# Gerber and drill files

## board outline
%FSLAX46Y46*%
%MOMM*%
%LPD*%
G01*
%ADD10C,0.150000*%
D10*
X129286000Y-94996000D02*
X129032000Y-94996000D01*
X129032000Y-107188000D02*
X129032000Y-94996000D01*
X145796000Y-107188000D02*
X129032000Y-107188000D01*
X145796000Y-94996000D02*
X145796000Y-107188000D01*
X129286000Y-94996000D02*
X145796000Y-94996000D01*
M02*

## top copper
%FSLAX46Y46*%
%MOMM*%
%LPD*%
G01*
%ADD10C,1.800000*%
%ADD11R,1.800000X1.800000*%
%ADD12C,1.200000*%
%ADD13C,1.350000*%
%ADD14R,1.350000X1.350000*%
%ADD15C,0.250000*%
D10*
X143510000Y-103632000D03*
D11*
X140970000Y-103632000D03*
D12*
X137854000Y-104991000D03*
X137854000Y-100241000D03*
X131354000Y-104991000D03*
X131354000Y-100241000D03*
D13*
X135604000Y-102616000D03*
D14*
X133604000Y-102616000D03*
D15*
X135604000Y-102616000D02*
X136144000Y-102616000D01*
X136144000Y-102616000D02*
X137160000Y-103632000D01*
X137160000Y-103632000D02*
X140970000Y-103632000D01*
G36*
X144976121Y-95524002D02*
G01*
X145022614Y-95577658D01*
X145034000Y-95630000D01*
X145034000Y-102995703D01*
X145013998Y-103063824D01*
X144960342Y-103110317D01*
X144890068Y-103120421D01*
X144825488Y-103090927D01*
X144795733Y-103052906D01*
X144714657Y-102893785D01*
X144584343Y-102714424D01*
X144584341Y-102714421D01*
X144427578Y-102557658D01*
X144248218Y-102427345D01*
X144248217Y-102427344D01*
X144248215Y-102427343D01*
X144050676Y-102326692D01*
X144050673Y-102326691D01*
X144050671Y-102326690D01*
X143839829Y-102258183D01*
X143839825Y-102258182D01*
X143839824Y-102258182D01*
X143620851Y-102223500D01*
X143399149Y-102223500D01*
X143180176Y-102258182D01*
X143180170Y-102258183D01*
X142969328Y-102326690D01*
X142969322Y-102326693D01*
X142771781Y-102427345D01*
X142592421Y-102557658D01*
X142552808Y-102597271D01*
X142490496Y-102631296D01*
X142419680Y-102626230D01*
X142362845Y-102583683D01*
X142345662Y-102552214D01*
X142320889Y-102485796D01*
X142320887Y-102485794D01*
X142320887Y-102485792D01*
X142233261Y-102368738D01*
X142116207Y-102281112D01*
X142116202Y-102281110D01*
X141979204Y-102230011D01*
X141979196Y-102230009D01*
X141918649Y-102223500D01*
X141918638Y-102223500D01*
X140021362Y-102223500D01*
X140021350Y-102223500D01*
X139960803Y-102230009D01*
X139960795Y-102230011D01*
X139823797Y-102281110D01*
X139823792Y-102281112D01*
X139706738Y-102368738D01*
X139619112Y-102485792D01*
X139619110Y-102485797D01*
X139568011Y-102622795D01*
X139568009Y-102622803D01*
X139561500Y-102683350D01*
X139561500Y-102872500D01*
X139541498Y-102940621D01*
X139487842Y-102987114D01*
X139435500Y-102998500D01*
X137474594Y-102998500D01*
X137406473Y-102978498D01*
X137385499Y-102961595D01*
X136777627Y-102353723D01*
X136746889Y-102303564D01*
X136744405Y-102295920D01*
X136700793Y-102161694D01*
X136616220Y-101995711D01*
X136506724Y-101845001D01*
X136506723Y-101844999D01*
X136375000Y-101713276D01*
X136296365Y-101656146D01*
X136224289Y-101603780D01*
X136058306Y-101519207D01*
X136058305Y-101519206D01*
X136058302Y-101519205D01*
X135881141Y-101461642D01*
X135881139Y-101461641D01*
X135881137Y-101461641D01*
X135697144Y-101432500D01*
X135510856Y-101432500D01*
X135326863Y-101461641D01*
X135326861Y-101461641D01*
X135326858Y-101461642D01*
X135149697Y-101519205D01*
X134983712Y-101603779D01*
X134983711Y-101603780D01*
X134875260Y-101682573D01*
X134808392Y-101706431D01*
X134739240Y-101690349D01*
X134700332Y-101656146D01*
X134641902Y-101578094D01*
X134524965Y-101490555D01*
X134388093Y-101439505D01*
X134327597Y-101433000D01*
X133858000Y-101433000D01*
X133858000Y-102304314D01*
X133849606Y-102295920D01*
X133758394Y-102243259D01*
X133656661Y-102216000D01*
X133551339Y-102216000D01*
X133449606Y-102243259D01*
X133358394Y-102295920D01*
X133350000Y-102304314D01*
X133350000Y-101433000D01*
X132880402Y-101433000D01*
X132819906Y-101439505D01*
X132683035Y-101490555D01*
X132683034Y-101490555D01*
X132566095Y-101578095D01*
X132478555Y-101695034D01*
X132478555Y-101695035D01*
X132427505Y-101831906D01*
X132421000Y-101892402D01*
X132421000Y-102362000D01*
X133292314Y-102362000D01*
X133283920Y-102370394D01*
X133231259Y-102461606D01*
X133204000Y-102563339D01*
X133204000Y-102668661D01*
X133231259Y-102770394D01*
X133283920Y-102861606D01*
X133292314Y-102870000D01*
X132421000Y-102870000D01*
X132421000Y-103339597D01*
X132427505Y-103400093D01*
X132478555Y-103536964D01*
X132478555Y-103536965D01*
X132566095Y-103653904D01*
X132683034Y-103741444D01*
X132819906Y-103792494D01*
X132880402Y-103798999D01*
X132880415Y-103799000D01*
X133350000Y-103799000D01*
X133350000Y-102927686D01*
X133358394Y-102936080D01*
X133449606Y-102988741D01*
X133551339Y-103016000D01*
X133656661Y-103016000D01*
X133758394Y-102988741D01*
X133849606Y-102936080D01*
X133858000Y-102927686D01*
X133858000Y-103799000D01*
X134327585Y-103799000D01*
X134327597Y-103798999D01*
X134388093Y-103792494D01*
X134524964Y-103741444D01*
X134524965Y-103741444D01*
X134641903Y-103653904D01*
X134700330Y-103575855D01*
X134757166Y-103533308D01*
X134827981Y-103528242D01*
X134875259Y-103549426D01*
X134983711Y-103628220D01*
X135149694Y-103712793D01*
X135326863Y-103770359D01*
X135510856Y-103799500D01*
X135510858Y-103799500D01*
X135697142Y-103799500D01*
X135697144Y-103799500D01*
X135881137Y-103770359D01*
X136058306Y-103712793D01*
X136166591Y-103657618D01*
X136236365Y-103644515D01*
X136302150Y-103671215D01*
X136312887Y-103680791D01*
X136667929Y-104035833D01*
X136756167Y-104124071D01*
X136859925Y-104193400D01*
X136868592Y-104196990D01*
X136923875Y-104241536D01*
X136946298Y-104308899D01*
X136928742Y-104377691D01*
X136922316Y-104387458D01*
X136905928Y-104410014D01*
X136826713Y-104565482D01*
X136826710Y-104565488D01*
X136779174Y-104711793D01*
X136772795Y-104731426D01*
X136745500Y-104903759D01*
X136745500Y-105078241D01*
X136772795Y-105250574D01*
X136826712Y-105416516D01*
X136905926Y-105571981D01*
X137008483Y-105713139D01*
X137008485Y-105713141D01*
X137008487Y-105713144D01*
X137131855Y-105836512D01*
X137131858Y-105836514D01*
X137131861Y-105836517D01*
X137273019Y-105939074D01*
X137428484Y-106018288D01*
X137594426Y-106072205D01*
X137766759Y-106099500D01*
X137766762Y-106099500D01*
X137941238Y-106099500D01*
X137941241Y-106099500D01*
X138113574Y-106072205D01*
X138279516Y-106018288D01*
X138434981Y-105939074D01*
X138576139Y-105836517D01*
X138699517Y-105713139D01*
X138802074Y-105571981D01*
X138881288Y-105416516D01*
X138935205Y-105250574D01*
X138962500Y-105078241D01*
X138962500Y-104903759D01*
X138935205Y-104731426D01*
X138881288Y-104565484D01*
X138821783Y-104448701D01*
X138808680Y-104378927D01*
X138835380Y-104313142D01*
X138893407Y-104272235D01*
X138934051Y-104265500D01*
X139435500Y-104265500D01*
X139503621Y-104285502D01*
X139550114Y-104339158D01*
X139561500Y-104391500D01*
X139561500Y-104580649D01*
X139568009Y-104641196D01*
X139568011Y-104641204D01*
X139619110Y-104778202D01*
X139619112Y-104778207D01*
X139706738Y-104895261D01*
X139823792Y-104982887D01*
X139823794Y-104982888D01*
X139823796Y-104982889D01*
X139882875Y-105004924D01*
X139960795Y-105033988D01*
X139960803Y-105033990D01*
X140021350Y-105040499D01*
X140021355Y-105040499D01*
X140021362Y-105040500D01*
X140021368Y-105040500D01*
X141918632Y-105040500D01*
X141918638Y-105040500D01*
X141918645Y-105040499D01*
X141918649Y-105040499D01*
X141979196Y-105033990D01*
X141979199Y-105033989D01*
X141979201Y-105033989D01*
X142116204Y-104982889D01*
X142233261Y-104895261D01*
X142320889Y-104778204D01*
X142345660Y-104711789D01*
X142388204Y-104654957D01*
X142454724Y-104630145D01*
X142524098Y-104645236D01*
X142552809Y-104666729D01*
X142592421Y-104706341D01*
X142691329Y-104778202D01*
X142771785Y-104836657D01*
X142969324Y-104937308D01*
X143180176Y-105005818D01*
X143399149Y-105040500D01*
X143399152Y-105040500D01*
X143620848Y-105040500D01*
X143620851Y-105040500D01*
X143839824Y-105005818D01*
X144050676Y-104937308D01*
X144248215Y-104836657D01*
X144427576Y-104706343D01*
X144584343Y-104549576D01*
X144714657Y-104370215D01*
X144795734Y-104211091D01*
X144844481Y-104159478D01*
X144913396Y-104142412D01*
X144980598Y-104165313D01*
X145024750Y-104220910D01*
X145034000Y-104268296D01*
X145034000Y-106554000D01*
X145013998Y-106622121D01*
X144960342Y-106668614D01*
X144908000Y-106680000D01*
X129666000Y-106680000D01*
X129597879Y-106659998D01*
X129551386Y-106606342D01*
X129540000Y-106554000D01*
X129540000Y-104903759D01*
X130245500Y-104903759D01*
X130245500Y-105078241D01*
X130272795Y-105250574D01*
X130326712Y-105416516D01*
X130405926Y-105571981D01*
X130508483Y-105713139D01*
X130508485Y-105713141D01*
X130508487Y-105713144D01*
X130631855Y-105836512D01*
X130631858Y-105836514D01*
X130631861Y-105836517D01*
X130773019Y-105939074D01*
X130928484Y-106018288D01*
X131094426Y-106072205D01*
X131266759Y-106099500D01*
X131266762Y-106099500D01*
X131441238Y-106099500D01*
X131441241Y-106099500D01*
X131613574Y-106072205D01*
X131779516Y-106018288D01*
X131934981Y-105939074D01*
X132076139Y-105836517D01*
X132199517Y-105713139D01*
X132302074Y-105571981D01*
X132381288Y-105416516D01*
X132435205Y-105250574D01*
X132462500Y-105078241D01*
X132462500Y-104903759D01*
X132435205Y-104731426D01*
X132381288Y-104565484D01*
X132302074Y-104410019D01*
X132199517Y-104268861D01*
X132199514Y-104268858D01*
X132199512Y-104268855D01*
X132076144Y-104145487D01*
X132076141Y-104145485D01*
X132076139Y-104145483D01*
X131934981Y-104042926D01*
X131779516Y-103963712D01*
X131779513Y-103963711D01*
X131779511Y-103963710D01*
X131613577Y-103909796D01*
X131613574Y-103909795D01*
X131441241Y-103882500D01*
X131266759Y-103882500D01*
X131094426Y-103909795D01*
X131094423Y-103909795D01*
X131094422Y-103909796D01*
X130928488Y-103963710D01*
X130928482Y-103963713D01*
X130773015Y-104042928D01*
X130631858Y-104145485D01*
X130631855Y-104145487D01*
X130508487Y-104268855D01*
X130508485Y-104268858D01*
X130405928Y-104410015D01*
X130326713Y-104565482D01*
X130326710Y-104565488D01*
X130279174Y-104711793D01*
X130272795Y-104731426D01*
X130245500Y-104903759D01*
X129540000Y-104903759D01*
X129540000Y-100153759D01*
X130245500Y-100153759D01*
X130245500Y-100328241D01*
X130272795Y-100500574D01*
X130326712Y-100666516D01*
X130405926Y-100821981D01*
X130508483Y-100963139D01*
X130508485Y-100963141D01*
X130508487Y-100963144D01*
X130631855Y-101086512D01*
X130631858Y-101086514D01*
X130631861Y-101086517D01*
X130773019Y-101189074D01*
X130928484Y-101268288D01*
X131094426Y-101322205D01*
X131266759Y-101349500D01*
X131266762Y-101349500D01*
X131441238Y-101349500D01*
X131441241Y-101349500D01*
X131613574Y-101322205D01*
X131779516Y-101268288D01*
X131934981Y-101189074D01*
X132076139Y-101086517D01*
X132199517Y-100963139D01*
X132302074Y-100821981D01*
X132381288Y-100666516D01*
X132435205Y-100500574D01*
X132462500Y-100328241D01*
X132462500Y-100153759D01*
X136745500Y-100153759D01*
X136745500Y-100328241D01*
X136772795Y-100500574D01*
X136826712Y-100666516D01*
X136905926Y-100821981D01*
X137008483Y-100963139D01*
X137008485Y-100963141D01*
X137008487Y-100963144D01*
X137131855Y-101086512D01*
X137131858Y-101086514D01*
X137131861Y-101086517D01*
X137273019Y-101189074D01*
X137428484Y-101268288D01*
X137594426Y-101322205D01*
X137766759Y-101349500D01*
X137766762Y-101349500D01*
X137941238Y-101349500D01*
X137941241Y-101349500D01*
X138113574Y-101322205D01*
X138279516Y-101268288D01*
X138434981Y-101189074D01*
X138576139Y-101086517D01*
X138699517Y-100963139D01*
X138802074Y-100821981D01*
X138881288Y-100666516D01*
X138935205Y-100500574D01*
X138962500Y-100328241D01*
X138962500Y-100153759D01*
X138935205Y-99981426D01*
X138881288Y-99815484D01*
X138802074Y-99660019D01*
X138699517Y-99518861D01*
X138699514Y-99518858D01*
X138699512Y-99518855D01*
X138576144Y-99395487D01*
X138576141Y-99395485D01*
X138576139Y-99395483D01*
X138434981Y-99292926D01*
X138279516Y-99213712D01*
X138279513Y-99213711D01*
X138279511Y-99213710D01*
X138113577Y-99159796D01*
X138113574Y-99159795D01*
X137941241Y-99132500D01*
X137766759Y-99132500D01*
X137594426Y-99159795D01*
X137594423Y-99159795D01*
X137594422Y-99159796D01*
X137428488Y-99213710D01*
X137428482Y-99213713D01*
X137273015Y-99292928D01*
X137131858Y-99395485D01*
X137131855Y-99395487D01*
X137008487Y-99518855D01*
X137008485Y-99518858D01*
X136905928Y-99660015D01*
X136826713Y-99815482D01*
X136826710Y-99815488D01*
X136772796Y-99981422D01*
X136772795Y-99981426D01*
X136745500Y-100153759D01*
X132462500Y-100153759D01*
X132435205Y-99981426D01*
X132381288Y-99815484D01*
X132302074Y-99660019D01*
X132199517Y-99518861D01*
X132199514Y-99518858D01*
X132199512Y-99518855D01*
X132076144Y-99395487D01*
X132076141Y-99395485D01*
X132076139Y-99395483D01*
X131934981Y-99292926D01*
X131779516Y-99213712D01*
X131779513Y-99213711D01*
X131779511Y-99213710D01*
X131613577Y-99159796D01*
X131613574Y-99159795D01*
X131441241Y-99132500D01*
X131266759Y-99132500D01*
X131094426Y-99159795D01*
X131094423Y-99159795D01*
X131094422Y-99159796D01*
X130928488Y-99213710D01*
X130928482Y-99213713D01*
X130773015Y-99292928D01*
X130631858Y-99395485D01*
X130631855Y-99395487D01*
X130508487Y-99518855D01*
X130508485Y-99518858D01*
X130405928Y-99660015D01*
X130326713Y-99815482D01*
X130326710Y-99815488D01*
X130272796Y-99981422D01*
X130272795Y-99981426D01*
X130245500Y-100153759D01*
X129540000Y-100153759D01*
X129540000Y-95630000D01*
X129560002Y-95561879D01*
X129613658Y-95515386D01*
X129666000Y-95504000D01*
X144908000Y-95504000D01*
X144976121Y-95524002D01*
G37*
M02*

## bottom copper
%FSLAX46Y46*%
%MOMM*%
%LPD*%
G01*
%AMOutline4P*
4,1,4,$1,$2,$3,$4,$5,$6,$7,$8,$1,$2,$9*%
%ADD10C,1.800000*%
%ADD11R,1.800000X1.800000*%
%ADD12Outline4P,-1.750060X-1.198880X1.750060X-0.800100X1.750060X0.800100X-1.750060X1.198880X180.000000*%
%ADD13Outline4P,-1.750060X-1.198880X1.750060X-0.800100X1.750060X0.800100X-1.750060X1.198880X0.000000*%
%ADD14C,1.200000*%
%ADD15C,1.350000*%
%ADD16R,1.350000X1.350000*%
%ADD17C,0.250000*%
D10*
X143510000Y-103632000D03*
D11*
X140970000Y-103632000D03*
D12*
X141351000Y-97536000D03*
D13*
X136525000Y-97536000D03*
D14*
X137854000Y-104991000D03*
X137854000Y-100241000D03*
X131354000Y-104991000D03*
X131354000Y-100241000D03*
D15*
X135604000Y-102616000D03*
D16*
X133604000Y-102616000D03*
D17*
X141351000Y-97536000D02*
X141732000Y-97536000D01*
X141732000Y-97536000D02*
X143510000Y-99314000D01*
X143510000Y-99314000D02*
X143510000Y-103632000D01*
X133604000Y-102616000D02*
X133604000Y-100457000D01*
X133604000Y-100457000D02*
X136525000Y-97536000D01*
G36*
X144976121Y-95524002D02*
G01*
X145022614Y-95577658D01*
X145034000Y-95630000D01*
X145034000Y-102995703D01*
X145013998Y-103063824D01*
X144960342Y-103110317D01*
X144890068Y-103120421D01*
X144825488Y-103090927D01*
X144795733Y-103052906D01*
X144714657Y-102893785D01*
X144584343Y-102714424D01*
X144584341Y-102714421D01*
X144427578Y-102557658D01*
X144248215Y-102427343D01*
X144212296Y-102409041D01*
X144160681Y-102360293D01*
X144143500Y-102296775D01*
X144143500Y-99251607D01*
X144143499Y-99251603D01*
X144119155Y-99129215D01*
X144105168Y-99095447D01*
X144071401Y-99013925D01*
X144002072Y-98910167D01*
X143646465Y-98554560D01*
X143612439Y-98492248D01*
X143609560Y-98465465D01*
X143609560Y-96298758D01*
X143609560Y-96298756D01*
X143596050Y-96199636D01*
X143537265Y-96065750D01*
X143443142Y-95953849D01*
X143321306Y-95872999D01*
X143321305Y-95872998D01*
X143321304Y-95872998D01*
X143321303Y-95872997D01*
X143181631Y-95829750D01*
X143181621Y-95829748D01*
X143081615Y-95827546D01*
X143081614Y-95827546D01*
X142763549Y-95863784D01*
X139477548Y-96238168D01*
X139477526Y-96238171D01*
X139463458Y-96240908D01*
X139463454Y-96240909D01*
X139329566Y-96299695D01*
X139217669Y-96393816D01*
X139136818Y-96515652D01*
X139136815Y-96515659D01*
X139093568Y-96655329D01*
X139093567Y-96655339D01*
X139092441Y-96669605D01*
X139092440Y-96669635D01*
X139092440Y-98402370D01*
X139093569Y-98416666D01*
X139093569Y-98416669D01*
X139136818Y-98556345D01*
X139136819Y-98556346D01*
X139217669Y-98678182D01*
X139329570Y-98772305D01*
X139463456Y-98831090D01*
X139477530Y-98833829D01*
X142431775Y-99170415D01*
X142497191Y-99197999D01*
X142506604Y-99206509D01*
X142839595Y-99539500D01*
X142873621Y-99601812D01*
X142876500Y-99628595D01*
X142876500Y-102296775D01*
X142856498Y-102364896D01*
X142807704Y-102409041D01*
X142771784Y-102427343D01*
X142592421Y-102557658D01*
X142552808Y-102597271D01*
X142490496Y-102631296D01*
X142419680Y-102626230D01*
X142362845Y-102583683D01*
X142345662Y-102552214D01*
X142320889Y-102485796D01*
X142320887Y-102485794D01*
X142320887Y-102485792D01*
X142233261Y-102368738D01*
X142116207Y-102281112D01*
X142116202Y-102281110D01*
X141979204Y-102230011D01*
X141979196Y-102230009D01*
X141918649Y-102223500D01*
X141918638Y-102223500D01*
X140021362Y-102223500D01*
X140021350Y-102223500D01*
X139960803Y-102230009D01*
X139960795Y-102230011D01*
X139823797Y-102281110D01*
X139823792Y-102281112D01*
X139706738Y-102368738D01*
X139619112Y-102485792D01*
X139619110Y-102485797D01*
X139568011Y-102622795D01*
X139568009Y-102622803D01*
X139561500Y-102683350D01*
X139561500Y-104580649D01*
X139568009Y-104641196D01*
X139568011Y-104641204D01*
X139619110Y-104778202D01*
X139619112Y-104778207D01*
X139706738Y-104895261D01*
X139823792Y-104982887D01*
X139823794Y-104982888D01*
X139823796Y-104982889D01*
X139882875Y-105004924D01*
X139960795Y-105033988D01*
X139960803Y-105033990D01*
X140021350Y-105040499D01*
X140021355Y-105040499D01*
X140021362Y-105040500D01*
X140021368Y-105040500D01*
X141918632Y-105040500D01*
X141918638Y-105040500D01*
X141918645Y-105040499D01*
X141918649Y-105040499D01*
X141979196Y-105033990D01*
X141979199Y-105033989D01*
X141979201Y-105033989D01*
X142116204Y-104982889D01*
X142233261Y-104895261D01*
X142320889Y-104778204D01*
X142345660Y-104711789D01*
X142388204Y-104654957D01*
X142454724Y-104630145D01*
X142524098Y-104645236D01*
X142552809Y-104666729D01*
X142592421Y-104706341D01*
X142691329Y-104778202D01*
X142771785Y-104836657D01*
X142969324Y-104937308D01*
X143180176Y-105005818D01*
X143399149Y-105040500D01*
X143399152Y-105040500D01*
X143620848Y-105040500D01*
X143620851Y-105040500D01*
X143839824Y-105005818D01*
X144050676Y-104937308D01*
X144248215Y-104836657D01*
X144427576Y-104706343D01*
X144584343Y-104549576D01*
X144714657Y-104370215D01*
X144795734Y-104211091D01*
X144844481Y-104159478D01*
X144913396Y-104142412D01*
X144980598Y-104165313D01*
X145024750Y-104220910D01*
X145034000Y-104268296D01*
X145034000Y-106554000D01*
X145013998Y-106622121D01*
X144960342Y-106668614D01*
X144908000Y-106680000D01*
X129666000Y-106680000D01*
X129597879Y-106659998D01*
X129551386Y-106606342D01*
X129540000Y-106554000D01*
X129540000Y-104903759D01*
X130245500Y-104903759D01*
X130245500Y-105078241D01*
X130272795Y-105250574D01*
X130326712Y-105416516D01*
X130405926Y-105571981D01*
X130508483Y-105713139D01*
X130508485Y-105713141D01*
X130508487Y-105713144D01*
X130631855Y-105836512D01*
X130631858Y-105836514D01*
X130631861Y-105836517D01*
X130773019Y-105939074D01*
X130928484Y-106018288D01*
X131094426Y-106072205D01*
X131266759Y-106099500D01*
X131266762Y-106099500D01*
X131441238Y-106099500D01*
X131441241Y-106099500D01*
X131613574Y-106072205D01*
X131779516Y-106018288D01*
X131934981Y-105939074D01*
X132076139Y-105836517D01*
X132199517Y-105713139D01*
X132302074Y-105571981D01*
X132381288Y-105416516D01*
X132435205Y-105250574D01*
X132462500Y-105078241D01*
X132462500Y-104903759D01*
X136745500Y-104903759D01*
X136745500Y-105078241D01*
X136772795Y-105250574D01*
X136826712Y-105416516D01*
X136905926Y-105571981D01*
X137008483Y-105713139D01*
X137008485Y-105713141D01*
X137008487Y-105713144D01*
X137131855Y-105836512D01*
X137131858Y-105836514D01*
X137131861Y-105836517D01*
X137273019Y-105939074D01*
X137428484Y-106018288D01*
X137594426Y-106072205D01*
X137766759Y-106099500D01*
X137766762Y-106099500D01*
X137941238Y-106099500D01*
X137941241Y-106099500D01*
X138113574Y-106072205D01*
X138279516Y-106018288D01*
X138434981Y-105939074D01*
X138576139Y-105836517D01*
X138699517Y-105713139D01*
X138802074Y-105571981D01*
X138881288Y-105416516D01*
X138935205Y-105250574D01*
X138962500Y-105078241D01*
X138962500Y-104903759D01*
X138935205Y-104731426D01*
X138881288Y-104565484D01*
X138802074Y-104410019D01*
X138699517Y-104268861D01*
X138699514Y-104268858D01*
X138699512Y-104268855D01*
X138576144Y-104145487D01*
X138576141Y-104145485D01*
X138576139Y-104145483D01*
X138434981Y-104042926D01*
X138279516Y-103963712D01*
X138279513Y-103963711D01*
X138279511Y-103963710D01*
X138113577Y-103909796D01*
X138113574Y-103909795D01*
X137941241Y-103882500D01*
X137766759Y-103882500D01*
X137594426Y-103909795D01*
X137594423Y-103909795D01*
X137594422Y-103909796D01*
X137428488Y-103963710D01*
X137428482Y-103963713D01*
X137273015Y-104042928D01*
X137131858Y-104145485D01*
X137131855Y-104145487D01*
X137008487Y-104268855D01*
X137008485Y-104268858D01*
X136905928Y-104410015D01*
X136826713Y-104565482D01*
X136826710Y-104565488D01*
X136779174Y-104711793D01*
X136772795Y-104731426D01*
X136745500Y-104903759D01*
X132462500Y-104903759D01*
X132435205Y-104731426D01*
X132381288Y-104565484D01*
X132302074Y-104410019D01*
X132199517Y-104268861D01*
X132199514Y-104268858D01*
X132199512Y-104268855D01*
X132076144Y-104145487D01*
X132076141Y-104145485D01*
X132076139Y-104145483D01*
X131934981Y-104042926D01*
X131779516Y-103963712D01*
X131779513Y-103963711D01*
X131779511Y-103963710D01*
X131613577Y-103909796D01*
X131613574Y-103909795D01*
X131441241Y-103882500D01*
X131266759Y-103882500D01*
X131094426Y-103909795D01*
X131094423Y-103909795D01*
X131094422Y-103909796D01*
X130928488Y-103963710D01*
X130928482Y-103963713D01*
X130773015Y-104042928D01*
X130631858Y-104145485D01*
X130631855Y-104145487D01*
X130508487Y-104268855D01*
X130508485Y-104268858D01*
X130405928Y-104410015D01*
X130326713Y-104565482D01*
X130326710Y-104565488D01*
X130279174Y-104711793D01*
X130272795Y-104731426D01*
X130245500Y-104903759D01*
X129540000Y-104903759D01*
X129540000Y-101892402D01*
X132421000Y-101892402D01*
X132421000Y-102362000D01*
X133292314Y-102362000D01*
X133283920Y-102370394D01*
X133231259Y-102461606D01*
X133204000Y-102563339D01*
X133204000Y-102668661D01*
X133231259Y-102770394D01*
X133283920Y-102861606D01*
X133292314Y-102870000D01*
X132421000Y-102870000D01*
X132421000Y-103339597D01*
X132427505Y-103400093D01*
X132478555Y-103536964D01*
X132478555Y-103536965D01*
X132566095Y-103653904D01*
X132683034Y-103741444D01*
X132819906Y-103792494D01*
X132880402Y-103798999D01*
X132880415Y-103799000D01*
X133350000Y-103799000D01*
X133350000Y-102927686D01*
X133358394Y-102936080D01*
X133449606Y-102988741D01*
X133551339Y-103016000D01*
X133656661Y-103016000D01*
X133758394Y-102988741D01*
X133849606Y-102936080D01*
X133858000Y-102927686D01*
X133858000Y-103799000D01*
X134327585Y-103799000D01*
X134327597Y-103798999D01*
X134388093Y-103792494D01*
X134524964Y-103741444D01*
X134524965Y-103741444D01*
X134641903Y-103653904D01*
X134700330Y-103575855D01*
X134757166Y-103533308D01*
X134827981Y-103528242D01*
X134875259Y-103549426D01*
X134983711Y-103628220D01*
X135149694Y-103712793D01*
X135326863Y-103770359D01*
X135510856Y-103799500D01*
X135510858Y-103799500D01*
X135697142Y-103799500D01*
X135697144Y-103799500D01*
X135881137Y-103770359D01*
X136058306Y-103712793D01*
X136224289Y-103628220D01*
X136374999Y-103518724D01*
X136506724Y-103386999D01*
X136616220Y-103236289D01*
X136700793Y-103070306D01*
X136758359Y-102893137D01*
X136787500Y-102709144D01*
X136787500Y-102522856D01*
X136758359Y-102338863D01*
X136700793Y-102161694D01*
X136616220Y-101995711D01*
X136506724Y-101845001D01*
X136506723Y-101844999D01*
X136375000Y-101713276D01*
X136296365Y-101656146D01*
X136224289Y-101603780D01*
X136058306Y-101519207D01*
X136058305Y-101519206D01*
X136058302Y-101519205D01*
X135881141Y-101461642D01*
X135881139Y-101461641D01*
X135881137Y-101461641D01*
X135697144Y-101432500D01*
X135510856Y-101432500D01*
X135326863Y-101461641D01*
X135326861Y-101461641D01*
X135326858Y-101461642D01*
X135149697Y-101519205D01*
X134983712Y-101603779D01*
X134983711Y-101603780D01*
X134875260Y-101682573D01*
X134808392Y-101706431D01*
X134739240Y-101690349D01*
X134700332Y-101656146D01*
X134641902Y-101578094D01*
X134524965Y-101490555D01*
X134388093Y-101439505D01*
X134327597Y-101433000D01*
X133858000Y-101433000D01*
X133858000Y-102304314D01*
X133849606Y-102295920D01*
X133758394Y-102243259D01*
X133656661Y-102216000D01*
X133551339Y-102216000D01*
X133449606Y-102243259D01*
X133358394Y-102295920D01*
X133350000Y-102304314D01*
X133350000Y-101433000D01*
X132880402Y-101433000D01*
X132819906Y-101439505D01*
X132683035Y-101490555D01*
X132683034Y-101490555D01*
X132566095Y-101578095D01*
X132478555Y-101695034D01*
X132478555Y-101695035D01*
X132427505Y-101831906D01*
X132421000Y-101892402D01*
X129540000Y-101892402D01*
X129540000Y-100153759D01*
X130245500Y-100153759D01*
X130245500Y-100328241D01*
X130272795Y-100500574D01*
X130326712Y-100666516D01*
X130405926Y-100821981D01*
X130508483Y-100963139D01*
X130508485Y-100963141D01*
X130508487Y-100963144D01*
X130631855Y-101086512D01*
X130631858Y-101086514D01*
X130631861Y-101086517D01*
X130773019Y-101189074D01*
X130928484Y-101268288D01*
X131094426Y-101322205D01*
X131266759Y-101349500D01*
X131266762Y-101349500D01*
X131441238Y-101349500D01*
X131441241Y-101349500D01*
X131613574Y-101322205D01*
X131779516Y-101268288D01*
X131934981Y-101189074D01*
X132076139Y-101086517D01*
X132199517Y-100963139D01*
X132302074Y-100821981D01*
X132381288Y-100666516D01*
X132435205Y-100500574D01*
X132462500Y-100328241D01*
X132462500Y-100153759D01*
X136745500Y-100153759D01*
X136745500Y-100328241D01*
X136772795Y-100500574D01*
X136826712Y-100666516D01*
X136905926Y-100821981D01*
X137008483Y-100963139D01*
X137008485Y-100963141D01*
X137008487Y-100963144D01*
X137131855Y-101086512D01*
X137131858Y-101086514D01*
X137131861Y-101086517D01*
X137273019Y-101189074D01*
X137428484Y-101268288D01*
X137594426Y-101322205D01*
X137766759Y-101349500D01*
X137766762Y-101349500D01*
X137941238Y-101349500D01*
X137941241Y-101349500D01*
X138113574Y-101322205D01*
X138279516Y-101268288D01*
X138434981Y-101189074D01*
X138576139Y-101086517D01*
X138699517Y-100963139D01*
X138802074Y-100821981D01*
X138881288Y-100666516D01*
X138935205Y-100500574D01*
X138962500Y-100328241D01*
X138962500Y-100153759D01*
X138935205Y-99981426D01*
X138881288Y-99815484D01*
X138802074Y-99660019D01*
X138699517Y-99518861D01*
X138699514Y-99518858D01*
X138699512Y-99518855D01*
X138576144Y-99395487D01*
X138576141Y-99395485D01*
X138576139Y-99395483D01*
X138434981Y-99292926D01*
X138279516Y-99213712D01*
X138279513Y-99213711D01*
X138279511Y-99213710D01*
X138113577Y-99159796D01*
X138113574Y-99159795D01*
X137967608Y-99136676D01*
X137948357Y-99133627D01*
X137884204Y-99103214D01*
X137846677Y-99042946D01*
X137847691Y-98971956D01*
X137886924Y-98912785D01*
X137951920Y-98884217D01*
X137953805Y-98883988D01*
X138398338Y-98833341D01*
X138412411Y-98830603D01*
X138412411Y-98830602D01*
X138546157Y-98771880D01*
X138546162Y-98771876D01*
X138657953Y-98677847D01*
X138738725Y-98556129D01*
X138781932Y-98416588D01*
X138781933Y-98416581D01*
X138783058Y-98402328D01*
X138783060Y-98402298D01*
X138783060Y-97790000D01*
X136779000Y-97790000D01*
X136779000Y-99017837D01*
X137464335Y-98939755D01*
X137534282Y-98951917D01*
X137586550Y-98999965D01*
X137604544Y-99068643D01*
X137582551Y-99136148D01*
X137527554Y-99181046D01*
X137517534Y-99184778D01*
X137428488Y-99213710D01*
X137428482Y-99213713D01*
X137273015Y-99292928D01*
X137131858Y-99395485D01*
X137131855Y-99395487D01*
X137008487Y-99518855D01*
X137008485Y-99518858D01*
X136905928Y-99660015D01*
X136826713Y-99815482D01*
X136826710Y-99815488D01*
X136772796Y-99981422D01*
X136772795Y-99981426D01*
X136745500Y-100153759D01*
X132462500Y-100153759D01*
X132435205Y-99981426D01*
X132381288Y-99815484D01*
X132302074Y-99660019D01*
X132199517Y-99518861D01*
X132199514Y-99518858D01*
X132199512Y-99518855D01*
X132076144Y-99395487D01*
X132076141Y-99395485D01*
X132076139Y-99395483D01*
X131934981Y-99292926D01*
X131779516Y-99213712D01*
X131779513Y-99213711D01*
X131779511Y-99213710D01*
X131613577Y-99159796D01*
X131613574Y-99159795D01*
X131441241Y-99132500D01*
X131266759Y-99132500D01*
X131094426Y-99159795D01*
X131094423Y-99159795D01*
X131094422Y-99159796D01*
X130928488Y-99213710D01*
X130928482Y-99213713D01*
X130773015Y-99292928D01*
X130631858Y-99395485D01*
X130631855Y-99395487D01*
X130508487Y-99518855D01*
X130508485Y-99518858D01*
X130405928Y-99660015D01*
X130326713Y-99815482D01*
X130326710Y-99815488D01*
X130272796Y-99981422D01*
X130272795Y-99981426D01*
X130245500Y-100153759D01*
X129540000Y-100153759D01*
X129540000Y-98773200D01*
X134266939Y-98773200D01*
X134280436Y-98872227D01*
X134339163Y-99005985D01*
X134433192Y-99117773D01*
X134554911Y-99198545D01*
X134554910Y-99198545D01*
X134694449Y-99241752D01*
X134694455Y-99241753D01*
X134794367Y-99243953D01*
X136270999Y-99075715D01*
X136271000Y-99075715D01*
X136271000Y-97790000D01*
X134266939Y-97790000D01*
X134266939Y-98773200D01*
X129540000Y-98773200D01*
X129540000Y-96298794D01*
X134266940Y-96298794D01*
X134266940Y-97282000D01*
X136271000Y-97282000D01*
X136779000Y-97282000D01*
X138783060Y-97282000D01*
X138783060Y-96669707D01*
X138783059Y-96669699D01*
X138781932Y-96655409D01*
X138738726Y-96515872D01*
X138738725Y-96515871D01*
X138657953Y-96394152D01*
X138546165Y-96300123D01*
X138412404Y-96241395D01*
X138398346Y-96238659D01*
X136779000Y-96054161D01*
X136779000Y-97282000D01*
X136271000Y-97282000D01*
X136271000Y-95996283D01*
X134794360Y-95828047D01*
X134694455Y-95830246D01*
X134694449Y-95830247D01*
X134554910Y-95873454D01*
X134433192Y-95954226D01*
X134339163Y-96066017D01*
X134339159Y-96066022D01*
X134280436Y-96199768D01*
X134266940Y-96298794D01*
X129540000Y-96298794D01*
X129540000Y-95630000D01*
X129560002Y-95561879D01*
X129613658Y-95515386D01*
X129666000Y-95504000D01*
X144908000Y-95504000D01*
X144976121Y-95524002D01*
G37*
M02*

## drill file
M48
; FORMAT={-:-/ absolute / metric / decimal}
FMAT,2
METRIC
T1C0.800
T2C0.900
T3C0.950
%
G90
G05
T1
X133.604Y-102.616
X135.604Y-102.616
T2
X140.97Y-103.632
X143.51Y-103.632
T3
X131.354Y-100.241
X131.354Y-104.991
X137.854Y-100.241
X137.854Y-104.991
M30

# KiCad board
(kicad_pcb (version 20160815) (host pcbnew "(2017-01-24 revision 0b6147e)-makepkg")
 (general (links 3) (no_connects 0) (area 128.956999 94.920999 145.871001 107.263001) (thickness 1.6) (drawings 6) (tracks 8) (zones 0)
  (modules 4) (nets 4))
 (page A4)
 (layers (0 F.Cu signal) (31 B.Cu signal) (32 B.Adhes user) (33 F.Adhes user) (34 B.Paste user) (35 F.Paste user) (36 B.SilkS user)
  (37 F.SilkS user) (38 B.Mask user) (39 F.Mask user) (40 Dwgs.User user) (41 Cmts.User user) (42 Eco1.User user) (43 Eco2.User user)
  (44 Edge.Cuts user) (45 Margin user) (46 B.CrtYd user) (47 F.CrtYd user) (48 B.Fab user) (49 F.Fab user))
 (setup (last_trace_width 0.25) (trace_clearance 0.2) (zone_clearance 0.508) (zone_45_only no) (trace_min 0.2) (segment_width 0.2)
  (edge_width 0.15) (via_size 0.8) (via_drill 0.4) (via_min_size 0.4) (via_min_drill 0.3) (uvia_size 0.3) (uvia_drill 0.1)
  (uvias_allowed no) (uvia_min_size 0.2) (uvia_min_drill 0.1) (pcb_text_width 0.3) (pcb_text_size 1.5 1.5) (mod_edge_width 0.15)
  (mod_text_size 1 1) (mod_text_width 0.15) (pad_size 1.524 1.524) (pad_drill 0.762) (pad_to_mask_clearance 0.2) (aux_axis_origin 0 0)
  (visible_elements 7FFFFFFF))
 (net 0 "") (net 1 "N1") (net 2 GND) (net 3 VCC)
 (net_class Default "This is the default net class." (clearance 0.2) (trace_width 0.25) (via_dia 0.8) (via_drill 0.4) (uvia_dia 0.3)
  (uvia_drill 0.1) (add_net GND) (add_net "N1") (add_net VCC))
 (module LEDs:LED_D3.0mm (layer F.Cu) (at 140.97 103.632)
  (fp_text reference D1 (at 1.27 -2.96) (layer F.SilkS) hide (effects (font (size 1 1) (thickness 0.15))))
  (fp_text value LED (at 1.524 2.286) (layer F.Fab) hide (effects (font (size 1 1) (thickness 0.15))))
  (pad 2 thru_hole circle (at 2.54 0) (size 1.8 1.8) (drill 0.9) (layers *.Cu *.Mask) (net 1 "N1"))
  (pad 1 thru_hole rect (at 0 0) (size 1.8 1.8) (drill 0.9) (layers *.Cu *.Mask) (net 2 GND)))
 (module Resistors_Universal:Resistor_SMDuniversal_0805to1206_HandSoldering (layer B.Cu) (at 138.938 97.536)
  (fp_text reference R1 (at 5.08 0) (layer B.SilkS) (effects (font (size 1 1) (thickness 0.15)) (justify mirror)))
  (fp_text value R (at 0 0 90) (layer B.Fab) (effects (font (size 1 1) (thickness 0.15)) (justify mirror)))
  (pad 2 smd trapezoid (at 2.413 0 180) (size 3.50012 1.99898) (rect_delta 0.39878 0) (layers B.Cu B.Paste B.Mask) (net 1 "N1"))
  (pad 1 smd trapezoid (at -2.413 0) (size 3.50012 1.99898) (rect_delta 0.39878 0) (layers B.Cu B.Paste B.Mask) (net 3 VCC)))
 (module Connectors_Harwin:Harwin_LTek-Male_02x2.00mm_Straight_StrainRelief (layer F.Cu) (at 133.604 102.616)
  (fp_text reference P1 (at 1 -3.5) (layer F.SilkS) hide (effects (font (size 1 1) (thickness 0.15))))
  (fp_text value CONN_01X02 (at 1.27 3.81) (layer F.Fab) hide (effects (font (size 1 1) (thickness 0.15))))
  (pad "" thru_hole circle (at 4.25 2.375) (size 1.2 1.2) (drill 0.95) (layers *.Cu *.Mask))
  (pad "" thru_hole circle (at 4.25 -2.375) (size 1.2 1.2) (drill 0.95) (layers *.Cu *.Mask))
  (pad "" thru_hole circle (at -2.25 2.375) (size 1.2 1.2) (drill 0.95) (layers *.Cu *.Mask))
  (pad "" thru_hole circle (at -2.25 -2.375) (size 1.2 1.2) (drill 0.95) (layers *.Cu *.Mask))
  (pad 2 thru_hole circle (at 2 0) (size 1.35 1.35) (drill 0.8) (layers *.Cu *.Mask) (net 2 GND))
  (pad 1 thru_hole rect (at 0 0) (size 1.35 1.35) (drill 0.8) (layers *.Cu *.Mask) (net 3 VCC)))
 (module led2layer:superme (layer F.Cu) (at 140.716 98.806)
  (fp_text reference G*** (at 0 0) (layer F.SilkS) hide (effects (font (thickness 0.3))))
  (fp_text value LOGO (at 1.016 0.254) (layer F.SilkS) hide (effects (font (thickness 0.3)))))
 (gr_line (start 129.286 94.996) (end 129.032 94.996) (angle 90) (layer Edge.Cuts) (width 0.15))
 (gr_line (start 129.032 107.188) (end 129.032 94.996) (angle 90) (layer Edge.Cuts) (width 0.15))
 (gr_line (start 145.796 107.188) (end 129.032 107.188) (angle 90) (layer Edge.Cuts) (width 0.15))
 (gr_line (start 145.796 94.996) (end 145.796 107.188) (angle 90) (layer Edge.Cuts) (width 0.15))
 (gr_line (start 129.286 94.996) (end 145.796 94.996) (angle 90) (layer Edge.Cuts) (width 0.15))
 (segment (start 141.351 97.536) (end 141.732 97.536) (width 0.25) (layer B.Cu) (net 1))
 (segment (start 141.732 97.536) (end 143.51 99.314) (width 0.25) (layer B.Cu) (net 1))
 (segment (start 143.51 99.314) (end 143.51 103.632) (width 0.25) (layer B.Cu) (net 1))
 (segment (start 135.604 102.616) (end 136.144 102.616) (width 0.25) (layer F.Cu) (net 2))
 (segment (start 136.144 102.616) (end 137.16 103.632) (width 0.25) (layer F.Cu) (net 2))
 (segment (start 137.16 103.632) (end 140.97 103.632) (width 0.25) (layer F.Cu) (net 2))
 (segment (start 133.604 102.616) (end 133.604 100.457) (width 0.25) (layer B.Cu) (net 3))
 (segment (start 133.604 100.457) (end 136.525 97.536) (width 0.25) (layer B.Cu) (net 3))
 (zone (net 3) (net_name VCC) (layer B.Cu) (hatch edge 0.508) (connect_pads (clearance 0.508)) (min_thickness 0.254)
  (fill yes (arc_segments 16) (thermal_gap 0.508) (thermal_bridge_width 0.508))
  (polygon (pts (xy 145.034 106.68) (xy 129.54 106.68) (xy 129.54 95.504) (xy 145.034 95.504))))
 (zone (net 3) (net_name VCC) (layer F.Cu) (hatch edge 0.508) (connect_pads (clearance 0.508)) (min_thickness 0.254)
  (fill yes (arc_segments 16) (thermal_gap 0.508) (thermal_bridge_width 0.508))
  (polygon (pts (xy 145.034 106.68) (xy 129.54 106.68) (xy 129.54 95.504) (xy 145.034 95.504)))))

